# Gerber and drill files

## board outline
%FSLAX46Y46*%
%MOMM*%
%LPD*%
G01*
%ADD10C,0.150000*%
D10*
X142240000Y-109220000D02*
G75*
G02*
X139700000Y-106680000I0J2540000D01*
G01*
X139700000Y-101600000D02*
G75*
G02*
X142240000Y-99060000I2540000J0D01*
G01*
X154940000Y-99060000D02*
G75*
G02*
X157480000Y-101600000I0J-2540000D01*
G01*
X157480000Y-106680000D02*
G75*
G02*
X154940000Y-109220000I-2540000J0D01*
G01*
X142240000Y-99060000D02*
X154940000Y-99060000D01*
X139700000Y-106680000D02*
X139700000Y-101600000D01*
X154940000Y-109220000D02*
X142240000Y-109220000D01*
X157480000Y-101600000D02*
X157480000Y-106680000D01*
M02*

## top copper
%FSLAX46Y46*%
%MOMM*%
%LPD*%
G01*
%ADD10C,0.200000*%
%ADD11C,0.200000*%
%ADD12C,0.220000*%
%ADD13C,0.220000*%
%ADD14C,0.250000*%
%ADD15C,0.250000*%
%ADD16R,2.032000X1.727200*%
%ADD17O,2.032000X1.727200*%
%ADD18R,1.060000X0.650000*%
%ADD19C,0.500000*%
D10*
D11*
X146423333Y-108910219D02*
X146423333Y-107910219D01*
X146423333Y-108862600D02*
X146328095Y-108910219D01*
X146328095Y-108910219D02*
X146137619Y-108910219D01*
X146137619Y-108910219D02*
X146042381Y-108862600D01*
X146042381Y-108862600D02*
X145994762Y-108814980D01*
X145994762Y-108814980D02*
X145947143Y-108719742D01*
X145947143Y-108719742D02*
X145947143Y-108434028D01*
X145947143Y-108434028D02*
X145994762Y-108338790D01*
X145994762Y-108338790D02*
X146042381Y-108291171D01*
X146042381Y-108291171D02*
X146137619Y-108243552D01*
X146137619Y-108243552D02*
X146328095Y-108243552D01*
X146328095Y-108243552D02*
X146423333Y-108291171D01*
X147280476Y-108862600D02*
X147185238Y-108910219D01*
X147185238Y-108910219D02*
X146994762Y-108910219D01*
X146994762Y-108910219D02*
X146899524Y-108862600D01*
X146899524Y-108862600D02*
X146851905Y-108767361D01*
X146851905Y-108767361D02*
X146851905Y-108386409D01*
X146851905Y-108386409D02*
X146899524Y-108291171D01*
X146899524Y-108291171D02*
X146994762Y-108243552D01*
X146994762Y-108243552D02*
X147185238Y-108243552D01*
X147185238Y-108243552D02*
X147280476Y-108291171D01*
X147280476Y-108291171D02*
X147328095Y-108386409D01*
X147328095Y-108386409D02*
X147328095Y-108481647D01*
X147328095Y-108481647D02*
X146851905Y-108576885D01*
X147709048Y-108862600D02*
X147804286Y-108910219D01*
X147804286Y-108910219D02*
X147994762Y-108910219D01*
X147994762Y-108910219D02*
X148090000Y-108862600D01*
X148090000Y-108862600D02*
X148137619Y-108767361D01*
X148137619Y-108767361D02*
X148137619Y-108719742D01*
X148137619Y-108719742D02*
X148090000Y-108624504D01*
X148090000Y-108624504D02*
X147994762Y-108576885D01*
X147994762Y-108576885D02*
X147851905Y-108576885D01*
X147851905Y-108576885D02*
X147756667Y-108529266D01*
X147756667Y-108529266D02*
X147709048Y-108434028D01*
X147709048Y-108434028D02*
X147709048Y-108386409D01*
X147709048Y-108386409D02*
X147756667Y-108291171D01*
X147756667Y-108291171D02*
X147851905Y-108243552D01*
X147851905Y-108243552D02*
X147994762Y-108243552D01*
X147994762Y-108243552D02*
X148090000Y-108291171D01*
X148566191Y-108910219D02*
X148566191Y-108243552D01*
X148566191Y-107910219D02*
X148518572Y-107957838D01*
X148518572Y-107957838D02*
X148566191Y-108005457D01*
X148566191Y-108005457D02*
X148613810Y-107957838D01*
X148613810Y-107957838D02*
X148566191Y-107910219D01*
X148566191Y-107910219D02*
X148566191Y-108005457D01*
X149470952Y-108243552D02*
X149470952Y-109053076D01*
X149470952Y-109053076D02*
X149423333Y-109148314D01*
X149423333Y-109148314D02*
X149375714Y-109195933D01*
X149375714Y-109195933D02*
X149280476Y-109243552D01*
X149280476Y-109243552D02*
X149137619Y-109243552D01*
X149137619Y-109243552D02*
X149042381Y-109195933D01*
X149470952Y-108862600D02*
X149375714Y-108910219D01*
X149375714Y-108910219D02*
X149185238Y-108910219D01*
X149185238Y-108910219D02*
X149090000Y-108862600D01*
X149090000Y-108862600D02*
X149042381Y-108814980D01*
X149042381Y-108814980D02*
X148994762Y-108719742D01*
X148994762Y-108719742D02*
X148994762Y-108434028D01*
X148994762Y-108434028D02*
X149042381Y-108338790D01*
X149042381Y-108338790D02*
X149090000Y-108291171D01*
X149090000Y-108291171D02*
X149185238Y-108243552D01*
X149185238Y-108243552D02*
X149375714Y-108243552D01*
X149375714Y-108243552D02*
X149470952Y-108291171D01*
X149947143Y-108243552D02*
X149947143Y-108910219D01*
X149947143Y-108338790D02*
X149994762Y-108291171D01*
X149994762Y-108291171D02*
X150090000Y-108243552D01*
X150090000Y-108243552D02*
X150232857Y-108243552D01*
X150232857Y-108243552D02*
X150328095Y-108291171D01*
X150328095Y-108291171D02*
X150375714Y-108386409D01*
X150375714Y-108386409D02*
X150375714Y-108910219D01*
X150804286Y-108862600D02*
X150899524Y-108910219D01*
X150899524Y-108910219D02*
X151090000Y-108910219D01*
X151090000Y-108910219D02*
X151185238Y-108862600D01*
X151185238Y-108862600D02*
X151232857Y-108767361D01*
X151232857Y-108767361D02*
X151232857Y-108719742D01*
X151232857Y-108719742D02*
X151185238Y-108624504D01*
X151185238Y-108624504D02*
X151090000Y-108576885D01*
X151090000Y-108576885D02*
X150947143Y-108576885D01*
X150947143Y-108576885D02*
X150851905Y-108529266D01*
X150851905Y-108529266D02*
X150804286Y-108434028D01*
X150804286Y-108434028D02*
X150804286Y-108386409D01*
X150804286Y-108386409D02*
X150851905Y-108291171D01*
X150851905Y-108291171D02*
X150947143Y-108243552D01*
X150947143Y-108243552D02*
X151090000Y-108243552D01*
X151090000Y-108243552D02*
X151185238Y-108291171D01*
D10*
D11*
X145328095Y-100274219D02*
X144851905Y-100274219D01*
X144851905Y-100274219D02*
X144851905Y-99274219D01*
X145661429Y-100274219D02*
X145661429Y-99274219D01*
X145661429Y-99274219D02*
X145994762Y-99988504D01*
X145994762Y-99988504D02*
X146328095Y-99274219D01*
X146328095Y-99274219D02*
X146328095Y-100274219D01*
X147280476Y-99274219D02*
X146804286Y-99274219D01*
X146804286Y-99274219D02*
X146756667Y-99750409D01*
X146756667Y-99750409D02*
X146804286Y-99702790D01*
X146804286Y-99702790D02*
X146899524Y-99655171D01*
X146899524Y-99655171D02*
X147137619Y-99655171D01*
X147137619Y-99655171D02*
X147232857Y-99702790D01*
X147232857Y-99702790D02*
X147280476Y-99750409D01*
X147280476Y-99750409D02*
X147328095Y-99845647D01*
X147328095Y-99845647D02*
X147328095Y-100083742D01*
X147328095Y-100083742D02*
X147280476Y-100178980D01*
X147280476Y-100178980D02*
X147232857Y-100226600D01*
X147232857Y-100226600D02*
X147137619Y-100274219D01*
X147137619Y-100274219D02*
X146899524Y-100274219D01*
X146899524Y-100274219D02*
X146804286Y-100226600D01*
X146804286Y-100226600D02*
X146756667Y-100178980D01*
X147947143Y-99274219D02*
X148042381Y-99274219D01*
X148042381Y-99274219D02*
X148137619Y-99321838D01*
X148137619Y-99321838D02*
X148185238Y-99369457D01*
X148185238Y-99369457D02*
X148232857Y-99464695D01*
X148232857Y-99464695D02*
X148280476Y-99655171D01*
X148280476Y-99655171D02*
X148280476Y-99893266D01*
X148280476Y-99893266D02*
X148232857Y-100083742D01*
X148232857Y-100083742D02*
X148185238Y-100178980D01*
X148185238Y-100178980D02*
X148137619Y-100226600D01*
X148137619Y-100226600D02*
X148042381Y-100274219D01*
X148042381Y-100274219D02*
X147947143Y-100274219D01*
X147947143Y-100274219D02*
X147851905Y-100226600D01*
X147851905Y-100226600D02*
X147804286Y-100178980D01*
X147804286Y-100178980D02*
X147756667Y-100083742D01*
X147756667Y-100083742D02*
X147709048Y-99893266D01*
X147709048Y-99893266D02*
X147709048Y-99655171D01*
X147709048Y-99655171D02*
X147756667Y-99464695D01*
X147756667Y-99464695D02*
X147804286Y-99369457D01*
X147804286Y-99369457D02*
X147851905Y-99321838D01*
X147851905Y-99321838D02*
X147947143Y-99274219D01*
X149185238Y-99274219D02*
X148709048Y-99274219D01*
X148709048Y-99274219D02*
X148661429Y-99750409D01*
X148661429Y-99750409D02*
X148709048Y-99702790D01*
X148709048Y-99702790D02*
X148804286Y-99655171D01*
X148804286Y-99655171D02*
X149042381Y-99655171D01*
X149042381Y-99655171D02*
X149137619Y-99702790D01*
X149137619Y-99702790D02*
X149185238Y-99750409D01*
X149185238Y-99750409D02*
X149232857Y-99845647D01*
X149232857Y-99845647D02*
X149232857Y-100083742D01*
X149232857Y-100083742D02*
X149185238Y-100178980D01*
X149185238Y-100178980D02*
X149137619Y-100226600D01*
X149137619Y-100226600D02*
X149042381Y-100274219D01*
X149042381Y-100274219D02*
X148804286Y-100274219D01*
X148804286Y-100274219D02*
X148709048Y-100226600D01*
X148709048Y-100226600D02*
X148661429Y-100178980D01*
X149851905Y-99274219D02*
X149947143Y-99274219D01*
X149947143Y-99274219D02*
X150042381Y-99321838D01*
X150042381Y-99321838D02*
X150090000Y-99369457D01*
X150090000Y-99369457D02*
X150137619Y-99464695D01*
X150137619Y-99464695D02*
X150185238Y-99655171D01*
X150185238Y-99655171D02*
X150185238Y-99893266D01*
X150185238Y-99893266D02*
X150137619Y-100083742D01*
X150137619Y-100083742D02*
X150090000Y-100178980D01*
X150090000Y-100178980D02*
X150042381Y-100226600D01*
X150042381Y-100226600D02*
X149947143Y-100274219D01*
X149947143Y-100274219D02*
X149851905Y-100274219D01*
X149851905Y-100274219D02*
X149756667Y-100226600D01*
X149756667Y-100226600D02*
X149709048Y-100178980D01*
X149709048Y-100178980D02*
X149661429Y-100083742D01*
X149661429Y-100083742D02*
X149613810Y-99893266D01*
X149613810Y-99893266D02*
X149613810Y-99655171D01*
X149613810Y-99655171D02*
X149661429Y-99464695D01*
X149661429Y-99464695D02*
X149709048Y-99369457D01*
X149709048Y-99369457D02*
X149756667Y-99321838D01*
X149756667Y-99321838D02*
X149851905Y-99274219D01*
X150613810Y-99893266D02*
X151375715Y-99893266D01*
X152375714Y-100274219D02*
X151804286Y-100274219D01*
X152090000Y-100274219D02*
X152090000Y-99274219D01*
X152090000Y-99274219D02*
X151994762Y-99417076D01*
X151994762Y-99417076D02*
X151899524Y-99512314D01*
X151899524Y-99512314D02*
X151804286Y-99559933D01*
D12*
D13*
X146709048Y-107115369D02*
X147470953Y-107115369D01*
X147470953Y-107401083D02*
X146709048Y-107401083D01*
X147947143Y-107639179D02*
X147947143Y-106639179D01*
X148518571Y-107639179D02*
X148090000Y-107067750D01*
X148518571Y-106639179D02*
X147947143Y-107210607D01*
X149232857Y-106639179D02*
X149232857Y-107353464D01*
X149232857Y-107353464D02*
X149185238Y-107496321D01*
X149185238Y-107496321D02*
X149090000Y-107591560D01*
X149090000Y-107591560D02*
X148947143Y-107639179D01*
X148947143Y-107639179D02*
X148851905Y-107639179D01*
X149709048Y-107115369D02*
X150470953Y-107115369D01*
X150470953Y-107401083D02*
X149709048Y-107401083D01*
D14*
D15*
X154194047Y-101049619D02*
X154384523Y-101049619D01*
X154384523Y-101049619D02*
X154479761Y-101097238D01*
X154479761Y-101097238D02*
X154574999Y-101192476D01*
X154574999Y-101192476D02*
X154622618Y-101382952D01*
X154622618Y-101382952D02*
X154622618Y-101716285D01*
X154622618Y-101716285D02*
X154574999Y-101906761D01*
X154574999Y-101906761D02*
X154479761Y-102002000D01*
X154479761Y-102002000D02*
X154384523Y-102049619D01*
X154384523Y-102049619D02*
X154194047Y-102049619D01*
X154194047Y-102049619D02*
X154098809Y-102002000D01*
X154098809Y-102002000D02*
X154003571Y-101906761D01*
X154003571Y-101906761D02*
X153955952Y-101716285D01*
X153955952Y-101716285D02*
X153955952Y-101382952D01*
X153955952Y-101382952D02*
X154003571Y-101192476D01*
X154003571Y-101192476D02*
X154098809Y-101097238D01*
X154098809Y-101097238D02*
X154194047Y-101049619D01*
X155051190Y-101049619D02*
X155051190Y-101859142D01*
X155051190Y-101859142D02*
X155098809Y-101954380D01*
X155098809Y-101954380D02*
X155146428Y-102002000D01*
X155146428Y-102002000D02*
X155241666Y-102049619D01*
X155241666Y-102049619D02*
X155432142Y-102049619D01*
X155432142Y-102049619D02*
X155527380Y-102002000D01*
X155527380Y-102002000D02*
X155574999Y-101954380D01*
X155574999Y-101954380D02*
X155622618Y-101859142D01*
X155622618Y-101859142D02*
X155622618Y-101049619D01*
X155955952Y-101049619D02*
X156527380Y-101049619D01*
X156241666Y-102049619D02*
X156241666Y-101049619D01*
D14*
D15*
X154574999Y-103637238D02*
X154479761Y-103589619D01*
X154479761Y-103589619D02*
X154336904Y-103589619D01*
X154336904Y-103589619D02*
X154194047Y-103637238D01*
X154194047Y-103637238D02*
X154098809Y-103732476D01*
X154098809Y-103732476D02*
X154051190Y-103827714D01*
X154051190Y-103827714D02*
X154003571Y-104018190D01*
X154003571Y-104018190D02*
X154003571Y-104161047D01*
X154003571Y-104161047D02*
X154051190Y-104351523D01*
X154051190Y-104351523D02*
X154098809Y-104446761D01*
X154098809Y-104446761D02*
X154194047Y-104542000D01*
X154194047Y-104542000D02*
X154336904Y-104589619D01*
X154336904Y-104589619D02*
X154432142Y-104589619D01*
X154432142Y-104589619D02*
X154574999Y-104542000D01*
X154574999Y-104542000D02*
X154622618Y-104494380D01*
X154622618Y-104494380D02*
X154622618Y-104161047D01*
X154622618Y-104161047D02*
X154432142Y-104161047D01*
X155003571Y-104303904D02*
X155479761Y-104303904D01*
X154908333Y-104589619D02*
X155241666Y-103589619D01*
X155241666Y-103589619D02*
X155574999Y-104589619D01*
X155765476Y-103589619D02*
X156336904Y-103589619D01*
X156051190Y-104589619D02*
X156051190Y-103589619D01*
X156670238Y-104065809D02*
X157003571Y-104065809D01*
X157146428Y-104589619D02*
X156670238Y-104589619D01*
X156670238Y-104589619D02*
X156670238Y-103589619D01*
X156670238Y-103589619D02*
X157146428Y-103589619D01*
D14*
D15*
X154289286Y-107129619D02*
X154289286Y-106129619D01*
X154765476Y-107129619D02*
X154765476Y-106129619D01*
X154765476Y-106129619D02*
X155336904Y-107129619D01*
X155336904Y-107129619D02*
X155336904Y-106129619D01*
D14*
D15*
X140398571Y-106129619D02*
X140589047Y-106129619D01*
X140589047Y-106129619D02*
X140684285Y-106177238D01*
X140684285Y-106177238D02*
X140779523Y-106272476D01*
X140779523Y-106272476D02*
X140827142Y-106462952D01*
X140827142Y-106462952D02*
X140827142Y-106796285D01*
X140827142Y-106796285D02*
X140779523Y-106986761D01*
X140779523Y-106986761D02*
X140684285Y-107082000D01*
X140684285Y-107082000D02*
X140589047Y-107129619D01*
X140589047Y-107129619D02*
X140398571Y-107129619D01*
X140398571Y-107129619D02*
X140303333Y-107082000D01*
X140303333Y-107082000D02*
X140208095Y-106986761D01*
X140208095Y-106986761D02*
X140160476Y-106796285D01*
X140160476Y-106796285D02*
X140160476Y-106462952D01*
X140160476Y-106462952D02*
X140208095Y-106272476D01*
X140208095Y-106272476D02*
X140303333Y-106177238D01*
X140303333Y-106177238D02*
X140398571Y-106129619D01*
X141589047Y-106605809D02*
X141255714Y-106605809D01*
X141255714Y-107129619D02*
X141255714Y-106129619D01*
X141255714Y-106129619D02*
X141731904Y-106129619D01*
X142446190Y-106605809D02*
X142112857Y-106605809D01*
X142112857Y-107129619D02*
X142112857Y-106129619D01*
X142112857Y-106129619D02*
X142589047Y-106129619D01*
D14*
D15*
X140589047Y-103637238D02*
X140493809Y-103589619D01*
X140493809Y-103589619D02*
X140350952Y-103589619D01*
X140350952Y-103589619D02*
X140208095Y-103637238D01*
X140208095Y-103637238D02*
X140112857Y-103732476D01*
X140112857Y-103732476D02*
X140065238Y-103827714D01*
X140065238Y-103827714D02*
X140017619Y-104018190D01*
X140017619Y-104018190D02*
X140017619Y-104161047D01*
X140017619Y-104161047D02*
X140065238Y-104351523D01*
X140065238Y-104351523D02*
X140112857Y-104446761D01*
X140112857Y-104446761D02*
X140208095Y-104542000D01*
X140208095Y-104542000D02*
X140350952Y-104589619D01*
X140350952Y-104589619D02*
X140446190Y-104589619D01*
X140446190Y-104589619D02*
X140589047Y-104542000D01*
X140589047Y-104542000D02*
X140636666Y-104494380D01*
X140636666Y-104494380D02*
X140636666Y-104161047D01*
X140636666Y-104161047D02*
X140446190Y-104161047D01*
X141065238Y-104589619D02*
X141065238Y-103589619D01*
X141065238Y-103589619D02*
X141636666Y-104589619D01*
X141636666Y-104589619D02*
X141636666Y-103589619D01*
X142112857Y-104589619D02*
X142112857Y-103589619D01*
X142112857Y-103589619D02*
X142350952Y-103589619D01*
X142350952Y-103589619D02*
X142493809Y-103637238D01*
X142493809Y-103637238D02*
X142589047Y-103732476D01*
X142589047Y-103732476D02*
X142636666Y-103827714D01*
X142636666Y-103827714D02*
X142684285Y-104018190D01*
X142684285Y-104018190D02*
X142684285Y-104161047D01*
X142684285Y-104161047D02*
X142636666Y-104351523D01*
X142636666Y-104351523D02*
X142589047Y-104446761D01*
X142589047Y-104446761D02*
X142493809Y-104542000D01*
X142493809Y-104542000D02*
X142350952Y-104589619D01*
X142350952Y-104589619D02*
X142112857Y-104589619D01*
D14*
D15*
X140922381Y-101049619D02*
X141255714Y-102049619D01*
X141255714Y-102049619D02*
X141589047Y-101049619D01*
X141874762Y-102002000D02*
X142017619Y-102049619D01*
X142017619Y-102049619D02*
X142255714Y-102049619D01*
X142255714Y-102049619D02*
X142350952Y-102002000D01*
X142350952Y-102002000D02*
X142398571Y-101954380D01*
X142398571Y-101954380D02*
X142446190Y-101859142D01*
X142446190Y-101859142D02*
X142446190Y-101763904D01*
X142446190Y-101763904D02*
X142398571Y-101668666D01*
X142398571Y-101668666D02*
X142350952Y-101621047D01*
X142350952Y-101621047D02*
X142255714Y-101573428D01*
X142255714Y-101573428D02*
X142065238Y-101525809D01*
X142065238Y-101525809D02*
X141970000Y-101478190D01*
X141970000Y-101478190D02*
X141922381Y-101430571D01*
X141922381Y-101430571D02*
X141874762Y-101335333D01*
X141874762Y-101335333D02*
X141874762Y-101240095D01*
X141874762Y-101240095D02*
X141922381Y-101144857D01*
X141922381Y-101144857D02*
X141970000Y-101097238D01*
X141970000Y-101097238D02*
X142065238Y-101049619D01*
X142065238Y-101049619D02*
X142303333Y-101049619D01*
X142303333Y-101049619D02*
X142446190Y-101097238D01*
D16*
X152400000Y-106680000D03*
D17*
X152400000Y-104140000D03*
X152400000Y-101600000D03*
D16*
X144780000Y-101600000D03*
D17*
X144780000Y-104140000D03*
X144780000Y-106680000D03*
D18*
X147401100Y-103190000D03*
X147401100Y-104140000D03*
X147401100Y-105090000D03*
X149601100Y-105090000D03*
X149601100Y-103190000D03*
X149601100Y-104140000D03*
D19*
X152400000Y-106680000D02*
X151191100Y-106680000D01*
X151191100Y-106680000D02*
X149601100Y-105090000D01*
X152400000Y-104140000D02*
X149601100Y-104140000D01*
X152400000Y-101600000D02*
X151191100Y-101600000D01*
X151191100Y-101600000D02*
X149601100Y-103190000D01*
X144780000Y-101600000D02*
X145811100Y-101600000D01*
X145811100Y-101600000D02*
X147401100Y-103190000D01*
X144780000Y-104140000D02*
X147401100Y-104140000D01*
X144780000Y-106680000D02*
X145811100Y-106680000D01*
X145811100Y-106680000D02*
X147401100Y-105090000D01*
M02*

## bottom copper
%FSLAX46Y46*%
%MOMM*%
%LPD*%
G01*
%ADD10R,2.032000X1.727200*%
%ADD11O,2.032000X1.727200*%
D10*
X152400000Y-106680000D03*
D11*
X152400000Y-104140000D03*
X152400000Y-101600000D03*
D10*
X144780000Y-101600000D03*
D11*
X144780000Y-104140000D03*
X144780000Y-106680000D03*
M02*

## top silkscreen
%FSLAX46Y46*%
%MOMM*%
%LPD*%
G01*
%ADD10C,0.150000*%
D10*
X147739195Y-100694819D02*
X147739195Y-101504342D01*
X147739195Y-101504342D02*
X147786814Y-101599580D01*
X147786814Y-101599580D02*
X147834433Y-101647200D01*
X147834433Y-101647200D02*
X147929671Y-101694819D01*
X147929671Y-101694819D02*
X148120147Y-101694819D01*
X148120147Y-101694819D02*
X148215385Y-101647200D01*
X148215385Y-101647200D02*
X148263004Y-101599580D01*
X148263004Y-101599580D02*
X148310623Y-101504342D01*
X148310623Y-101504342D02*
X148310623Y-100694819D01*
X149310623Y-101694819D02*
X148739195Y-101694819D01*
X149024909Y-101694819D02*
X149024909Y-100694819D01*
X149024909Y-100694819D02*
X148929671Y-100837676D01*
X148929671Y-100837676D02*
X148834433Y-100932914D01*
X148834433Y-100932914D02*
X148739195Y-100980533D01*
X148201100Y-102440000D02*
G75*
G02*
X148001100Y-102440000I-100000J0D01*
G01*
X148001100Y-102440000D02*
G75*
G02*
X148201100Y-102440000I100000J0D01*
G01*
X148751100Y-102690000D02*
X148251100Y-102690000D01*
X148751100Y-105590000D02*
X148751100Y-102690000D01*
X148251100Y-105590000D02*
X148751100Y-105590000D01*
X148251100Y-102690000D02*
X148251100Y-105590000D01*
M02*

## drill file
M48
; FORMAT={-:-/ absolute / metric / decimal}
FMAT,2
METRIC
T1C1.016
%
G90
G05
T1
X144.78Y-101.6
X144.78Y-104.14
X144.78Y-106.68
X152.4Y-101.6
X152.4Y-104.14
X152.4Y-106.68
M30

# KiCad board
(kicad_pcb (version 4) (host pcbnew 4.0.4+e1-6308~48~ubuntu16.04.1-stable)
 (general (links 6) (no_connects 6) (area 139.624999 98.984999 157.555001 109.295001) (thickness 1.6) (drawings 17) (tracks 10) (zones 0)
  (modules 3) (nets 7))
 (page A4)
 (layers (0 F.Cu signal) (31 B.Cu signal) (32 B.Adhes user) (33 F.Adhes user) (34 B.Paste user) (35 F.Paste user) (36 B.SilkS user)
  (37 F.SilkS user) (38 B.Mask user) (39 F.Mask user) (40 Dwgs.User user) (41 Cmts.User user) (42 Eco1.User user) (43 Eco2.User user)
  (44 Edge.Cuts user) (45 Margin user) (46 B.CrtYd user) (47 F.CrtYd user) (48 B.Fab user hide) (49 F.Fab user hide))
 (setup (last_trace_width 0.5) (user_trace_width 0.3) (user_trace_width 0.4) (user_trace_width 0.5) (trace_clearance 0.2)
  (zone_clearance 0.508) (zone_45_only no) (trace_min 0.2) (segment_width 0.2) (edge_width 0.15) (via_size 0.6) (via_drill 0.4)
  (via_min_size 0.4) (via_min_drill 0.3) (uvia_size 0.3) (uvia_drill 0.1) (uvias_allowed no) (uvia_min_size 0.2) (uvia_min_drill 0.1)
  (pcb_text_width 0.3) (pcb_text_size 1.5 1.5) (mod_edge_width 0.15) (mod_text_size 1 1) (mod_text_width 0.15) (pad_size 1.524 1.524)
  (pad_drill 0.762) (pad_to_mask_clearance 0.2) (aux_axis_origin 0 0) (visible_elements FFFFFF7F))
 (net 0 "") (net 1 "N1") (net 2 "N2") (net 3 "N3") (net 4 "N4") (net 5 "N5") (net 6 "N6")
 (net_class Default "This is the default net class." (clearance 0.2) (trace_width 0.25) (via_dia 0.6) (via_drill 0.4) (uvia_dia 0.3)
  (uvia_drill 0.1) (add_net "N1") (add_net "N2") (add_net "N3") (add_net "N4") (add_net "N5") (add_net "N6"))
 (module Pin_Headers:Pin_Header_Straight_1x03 (layer B.Cu) (at 152.4 106.68)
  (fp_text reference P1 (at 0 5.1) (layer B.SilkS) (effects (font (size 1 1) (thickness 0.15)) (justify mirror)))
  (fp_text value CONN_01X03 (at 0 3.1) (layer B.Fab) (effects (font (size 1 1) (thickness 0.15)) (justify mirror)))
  (pad 1 thru_hole rect (at 0 0) (size 2.032 1.7272) (drill 1.016) (layers *.Cu *.Mask) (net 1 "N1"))
  (pad 2 thru_hole oval (at 0 -2.54) (size 2.032 1.7272) (drill 1.016) (layers *.Cu *.Mask) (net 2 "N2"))
  (pad 3 thru_hole oval (at 0 -5.08) (size 2.032 1.7272) (drill 1.016) (layers *.Cu *.Mask) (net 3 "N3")))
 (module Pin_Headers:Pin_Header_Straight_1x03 (layer B.Cu) (at 144.78 101.6 180)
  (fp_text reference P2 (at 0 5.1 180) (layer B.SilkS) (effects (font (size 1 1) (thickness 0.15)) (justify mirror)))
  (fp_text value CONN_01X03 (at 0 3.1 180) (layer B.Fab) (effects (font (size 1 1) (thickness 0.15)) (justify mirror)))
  (pad 1 thru_hole rect (at 0 0 180) (size 2.032 1.7272) (drill 1.016) (layers *.Cu *.Mask) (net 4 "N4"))
  (pad 2 thru_hole oval (at 0 -2.54 180) (size 2.032 1.7272) (drill 1.016) (layers *.Cu *.Mask) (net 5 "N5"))
  (pad 3 thru_hole oval (at 0 -5.08 180) (size 2.032 1.7272) (drill 1.016) (layers *.Cu *.Mask) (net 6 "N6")))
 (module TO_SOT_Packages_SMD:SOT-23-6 (layer F.Cu) (at 148.5011 104.14)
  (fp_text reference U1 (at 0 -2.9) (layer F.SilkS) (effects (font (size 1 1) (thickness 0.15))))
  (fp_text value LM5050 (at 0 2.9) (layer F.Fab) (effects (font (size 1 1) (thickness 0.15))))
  (fp_circle (center -0.4 -1.7) (end -0.3 -1.7) (layer F.SilkS) (width 0.15))
  (fp_line (start 0.25 -1.45) (end -0.25 -1.45) (layer F.SilkS) (width 0.15))
  (fp_line (start 0.25 1.45) (end 0.25 -1.45) (layer F.SilkS) (width 0.15))
  (fp_line (start -0.25 1.45) (end 0.25 1.45) (layer F.SilkS) (width 0.15))
  (fp_line (start -0.25 -1.45) (end -0.25 1.45) (layer F.SilkS) (width 0.15))
  (pad 1 smd rect (at -1.1 -0.95) (size 1.06 0.65) (layers F.Cu F.Paste F.Mask) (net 4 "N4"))
  (pad 2 smd rect (at -1.1 0) (size 1.06 0.65) (layers F.Cu F.Paste F.Mask) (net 5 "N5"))
  (pad 3 smd rect (at -1.1 0.95) (size 1.06 0.65) (layers F.Cu F.Paste F.Mask) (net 6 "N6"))
  (pad 4 smd rect (at 1.1 0.95) (size 1.06 0.65) (layers F.Cu F.Paste F.Mask) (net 1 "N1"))
  (pad 6 smd rect (at 1.1 -0.95) (size 1.06 0.65) (layers F.Cu F.Paste F.Mask) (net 3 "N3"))
  (pad 5 smd rect (at 1.1 0) (size 1.06 0.65) (layers F.Cu F.Paste F.Mask) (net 2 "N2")))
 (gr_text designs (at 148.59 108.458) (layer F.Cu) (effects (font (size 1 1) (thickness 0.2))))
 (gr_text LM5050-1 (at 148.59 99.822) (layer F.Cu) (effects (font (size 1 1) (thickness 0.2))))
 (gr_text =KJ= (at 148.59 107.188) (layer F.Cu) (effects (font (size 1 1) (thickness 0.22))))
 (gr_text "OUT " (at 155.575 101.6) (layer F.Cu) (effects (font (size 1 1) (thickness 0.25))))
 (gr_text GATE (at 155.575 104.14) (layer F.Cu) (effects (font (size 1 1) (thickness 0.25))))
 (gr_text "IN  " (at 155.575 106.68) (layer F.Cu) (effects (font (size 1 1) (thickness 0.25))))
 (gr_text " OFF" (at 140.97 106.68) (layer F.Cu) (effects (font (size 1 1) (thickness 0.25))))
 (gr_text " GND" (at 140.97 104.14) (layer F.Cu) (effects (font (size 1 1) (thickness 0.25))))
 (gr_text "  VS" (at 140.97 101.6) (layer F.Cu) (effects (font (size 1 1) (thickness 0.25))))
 (gr_arc (start 142.24 106.68) (end 142.24 109.22) (angle 90) (layer Edge.Cuts) (width 0.15))
 (gr_arc (start 142.24 101.6) (end 139.7 101.6) (angle 90) (layer Edge.Cuts) (width 0.15))
 (gr_arc (start 154.94 101.6) (end 154.94 99.06) (angle 90) (layer Edge.Cuts) (width 0.15))
 (gr_arc (start 154.94 106.68) (end 157.48 106.68) (angle 90) (layer Edge.Cuts) (width 0.15))
 (gr_line (start 142.24 99.06) (end 154.94 99.06) (layer Edge.Cuts) (width 0.15))
 (gr_line (start 139.7 106.68) (end 139.7 101.6) (layer Edge.Cuts) (width 0.15))
 (gr_line (start 154.94 109.22) (end 142.24 109.22) (layer Edge.Cuts) (width 0.15))
 (gr_line (start 157.48 101.6) (end 157.48 106.68) (layer Edge.Cuts) (width 0.15))
 (segment (start 152.4 106.68) (end 151.1911 106.68) (width 0.5) (layer F.Cu) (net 1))
 (segment (start 151.1911 106.68) (end 149.6011 105.09) (width 0.5) (layer F.Cu) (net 1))
 (segment (start 152.4 104.14) (end 149.6011 104.14) (width 0.5) (layer F.Cu) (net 2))
 (segment (start 152.4 101.6) (end 151.1911 101.6) (width 0.5) (layer F.Cu) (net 3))
 (segment (start 151.1911 101.6) (end 149.6011 103.19) (width 0.5) (layer F.Cu) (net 3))
 (segment (start 144.78 101.6) (end 145.8111 101.6) (width 0.5) (layer F.Cu) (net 4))
 (segment (start 145.8111 101.6) (end 147.4011 103.19) (width 0.5) (layer F.Cu) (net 4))
 (segment (start 144.78 104.14) (end 147.4011 104.14) (width 0.5) (layer F.Cu) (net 5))
 (segment (start 144.78 106.68) (end 145.8111 106.68) (width 0.5) (layer F.Cu) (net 6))
 (segment (start 145.8111 106.68) (end 147.4011 105.09) (width 0.5) (layer F.Cu) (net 6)))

